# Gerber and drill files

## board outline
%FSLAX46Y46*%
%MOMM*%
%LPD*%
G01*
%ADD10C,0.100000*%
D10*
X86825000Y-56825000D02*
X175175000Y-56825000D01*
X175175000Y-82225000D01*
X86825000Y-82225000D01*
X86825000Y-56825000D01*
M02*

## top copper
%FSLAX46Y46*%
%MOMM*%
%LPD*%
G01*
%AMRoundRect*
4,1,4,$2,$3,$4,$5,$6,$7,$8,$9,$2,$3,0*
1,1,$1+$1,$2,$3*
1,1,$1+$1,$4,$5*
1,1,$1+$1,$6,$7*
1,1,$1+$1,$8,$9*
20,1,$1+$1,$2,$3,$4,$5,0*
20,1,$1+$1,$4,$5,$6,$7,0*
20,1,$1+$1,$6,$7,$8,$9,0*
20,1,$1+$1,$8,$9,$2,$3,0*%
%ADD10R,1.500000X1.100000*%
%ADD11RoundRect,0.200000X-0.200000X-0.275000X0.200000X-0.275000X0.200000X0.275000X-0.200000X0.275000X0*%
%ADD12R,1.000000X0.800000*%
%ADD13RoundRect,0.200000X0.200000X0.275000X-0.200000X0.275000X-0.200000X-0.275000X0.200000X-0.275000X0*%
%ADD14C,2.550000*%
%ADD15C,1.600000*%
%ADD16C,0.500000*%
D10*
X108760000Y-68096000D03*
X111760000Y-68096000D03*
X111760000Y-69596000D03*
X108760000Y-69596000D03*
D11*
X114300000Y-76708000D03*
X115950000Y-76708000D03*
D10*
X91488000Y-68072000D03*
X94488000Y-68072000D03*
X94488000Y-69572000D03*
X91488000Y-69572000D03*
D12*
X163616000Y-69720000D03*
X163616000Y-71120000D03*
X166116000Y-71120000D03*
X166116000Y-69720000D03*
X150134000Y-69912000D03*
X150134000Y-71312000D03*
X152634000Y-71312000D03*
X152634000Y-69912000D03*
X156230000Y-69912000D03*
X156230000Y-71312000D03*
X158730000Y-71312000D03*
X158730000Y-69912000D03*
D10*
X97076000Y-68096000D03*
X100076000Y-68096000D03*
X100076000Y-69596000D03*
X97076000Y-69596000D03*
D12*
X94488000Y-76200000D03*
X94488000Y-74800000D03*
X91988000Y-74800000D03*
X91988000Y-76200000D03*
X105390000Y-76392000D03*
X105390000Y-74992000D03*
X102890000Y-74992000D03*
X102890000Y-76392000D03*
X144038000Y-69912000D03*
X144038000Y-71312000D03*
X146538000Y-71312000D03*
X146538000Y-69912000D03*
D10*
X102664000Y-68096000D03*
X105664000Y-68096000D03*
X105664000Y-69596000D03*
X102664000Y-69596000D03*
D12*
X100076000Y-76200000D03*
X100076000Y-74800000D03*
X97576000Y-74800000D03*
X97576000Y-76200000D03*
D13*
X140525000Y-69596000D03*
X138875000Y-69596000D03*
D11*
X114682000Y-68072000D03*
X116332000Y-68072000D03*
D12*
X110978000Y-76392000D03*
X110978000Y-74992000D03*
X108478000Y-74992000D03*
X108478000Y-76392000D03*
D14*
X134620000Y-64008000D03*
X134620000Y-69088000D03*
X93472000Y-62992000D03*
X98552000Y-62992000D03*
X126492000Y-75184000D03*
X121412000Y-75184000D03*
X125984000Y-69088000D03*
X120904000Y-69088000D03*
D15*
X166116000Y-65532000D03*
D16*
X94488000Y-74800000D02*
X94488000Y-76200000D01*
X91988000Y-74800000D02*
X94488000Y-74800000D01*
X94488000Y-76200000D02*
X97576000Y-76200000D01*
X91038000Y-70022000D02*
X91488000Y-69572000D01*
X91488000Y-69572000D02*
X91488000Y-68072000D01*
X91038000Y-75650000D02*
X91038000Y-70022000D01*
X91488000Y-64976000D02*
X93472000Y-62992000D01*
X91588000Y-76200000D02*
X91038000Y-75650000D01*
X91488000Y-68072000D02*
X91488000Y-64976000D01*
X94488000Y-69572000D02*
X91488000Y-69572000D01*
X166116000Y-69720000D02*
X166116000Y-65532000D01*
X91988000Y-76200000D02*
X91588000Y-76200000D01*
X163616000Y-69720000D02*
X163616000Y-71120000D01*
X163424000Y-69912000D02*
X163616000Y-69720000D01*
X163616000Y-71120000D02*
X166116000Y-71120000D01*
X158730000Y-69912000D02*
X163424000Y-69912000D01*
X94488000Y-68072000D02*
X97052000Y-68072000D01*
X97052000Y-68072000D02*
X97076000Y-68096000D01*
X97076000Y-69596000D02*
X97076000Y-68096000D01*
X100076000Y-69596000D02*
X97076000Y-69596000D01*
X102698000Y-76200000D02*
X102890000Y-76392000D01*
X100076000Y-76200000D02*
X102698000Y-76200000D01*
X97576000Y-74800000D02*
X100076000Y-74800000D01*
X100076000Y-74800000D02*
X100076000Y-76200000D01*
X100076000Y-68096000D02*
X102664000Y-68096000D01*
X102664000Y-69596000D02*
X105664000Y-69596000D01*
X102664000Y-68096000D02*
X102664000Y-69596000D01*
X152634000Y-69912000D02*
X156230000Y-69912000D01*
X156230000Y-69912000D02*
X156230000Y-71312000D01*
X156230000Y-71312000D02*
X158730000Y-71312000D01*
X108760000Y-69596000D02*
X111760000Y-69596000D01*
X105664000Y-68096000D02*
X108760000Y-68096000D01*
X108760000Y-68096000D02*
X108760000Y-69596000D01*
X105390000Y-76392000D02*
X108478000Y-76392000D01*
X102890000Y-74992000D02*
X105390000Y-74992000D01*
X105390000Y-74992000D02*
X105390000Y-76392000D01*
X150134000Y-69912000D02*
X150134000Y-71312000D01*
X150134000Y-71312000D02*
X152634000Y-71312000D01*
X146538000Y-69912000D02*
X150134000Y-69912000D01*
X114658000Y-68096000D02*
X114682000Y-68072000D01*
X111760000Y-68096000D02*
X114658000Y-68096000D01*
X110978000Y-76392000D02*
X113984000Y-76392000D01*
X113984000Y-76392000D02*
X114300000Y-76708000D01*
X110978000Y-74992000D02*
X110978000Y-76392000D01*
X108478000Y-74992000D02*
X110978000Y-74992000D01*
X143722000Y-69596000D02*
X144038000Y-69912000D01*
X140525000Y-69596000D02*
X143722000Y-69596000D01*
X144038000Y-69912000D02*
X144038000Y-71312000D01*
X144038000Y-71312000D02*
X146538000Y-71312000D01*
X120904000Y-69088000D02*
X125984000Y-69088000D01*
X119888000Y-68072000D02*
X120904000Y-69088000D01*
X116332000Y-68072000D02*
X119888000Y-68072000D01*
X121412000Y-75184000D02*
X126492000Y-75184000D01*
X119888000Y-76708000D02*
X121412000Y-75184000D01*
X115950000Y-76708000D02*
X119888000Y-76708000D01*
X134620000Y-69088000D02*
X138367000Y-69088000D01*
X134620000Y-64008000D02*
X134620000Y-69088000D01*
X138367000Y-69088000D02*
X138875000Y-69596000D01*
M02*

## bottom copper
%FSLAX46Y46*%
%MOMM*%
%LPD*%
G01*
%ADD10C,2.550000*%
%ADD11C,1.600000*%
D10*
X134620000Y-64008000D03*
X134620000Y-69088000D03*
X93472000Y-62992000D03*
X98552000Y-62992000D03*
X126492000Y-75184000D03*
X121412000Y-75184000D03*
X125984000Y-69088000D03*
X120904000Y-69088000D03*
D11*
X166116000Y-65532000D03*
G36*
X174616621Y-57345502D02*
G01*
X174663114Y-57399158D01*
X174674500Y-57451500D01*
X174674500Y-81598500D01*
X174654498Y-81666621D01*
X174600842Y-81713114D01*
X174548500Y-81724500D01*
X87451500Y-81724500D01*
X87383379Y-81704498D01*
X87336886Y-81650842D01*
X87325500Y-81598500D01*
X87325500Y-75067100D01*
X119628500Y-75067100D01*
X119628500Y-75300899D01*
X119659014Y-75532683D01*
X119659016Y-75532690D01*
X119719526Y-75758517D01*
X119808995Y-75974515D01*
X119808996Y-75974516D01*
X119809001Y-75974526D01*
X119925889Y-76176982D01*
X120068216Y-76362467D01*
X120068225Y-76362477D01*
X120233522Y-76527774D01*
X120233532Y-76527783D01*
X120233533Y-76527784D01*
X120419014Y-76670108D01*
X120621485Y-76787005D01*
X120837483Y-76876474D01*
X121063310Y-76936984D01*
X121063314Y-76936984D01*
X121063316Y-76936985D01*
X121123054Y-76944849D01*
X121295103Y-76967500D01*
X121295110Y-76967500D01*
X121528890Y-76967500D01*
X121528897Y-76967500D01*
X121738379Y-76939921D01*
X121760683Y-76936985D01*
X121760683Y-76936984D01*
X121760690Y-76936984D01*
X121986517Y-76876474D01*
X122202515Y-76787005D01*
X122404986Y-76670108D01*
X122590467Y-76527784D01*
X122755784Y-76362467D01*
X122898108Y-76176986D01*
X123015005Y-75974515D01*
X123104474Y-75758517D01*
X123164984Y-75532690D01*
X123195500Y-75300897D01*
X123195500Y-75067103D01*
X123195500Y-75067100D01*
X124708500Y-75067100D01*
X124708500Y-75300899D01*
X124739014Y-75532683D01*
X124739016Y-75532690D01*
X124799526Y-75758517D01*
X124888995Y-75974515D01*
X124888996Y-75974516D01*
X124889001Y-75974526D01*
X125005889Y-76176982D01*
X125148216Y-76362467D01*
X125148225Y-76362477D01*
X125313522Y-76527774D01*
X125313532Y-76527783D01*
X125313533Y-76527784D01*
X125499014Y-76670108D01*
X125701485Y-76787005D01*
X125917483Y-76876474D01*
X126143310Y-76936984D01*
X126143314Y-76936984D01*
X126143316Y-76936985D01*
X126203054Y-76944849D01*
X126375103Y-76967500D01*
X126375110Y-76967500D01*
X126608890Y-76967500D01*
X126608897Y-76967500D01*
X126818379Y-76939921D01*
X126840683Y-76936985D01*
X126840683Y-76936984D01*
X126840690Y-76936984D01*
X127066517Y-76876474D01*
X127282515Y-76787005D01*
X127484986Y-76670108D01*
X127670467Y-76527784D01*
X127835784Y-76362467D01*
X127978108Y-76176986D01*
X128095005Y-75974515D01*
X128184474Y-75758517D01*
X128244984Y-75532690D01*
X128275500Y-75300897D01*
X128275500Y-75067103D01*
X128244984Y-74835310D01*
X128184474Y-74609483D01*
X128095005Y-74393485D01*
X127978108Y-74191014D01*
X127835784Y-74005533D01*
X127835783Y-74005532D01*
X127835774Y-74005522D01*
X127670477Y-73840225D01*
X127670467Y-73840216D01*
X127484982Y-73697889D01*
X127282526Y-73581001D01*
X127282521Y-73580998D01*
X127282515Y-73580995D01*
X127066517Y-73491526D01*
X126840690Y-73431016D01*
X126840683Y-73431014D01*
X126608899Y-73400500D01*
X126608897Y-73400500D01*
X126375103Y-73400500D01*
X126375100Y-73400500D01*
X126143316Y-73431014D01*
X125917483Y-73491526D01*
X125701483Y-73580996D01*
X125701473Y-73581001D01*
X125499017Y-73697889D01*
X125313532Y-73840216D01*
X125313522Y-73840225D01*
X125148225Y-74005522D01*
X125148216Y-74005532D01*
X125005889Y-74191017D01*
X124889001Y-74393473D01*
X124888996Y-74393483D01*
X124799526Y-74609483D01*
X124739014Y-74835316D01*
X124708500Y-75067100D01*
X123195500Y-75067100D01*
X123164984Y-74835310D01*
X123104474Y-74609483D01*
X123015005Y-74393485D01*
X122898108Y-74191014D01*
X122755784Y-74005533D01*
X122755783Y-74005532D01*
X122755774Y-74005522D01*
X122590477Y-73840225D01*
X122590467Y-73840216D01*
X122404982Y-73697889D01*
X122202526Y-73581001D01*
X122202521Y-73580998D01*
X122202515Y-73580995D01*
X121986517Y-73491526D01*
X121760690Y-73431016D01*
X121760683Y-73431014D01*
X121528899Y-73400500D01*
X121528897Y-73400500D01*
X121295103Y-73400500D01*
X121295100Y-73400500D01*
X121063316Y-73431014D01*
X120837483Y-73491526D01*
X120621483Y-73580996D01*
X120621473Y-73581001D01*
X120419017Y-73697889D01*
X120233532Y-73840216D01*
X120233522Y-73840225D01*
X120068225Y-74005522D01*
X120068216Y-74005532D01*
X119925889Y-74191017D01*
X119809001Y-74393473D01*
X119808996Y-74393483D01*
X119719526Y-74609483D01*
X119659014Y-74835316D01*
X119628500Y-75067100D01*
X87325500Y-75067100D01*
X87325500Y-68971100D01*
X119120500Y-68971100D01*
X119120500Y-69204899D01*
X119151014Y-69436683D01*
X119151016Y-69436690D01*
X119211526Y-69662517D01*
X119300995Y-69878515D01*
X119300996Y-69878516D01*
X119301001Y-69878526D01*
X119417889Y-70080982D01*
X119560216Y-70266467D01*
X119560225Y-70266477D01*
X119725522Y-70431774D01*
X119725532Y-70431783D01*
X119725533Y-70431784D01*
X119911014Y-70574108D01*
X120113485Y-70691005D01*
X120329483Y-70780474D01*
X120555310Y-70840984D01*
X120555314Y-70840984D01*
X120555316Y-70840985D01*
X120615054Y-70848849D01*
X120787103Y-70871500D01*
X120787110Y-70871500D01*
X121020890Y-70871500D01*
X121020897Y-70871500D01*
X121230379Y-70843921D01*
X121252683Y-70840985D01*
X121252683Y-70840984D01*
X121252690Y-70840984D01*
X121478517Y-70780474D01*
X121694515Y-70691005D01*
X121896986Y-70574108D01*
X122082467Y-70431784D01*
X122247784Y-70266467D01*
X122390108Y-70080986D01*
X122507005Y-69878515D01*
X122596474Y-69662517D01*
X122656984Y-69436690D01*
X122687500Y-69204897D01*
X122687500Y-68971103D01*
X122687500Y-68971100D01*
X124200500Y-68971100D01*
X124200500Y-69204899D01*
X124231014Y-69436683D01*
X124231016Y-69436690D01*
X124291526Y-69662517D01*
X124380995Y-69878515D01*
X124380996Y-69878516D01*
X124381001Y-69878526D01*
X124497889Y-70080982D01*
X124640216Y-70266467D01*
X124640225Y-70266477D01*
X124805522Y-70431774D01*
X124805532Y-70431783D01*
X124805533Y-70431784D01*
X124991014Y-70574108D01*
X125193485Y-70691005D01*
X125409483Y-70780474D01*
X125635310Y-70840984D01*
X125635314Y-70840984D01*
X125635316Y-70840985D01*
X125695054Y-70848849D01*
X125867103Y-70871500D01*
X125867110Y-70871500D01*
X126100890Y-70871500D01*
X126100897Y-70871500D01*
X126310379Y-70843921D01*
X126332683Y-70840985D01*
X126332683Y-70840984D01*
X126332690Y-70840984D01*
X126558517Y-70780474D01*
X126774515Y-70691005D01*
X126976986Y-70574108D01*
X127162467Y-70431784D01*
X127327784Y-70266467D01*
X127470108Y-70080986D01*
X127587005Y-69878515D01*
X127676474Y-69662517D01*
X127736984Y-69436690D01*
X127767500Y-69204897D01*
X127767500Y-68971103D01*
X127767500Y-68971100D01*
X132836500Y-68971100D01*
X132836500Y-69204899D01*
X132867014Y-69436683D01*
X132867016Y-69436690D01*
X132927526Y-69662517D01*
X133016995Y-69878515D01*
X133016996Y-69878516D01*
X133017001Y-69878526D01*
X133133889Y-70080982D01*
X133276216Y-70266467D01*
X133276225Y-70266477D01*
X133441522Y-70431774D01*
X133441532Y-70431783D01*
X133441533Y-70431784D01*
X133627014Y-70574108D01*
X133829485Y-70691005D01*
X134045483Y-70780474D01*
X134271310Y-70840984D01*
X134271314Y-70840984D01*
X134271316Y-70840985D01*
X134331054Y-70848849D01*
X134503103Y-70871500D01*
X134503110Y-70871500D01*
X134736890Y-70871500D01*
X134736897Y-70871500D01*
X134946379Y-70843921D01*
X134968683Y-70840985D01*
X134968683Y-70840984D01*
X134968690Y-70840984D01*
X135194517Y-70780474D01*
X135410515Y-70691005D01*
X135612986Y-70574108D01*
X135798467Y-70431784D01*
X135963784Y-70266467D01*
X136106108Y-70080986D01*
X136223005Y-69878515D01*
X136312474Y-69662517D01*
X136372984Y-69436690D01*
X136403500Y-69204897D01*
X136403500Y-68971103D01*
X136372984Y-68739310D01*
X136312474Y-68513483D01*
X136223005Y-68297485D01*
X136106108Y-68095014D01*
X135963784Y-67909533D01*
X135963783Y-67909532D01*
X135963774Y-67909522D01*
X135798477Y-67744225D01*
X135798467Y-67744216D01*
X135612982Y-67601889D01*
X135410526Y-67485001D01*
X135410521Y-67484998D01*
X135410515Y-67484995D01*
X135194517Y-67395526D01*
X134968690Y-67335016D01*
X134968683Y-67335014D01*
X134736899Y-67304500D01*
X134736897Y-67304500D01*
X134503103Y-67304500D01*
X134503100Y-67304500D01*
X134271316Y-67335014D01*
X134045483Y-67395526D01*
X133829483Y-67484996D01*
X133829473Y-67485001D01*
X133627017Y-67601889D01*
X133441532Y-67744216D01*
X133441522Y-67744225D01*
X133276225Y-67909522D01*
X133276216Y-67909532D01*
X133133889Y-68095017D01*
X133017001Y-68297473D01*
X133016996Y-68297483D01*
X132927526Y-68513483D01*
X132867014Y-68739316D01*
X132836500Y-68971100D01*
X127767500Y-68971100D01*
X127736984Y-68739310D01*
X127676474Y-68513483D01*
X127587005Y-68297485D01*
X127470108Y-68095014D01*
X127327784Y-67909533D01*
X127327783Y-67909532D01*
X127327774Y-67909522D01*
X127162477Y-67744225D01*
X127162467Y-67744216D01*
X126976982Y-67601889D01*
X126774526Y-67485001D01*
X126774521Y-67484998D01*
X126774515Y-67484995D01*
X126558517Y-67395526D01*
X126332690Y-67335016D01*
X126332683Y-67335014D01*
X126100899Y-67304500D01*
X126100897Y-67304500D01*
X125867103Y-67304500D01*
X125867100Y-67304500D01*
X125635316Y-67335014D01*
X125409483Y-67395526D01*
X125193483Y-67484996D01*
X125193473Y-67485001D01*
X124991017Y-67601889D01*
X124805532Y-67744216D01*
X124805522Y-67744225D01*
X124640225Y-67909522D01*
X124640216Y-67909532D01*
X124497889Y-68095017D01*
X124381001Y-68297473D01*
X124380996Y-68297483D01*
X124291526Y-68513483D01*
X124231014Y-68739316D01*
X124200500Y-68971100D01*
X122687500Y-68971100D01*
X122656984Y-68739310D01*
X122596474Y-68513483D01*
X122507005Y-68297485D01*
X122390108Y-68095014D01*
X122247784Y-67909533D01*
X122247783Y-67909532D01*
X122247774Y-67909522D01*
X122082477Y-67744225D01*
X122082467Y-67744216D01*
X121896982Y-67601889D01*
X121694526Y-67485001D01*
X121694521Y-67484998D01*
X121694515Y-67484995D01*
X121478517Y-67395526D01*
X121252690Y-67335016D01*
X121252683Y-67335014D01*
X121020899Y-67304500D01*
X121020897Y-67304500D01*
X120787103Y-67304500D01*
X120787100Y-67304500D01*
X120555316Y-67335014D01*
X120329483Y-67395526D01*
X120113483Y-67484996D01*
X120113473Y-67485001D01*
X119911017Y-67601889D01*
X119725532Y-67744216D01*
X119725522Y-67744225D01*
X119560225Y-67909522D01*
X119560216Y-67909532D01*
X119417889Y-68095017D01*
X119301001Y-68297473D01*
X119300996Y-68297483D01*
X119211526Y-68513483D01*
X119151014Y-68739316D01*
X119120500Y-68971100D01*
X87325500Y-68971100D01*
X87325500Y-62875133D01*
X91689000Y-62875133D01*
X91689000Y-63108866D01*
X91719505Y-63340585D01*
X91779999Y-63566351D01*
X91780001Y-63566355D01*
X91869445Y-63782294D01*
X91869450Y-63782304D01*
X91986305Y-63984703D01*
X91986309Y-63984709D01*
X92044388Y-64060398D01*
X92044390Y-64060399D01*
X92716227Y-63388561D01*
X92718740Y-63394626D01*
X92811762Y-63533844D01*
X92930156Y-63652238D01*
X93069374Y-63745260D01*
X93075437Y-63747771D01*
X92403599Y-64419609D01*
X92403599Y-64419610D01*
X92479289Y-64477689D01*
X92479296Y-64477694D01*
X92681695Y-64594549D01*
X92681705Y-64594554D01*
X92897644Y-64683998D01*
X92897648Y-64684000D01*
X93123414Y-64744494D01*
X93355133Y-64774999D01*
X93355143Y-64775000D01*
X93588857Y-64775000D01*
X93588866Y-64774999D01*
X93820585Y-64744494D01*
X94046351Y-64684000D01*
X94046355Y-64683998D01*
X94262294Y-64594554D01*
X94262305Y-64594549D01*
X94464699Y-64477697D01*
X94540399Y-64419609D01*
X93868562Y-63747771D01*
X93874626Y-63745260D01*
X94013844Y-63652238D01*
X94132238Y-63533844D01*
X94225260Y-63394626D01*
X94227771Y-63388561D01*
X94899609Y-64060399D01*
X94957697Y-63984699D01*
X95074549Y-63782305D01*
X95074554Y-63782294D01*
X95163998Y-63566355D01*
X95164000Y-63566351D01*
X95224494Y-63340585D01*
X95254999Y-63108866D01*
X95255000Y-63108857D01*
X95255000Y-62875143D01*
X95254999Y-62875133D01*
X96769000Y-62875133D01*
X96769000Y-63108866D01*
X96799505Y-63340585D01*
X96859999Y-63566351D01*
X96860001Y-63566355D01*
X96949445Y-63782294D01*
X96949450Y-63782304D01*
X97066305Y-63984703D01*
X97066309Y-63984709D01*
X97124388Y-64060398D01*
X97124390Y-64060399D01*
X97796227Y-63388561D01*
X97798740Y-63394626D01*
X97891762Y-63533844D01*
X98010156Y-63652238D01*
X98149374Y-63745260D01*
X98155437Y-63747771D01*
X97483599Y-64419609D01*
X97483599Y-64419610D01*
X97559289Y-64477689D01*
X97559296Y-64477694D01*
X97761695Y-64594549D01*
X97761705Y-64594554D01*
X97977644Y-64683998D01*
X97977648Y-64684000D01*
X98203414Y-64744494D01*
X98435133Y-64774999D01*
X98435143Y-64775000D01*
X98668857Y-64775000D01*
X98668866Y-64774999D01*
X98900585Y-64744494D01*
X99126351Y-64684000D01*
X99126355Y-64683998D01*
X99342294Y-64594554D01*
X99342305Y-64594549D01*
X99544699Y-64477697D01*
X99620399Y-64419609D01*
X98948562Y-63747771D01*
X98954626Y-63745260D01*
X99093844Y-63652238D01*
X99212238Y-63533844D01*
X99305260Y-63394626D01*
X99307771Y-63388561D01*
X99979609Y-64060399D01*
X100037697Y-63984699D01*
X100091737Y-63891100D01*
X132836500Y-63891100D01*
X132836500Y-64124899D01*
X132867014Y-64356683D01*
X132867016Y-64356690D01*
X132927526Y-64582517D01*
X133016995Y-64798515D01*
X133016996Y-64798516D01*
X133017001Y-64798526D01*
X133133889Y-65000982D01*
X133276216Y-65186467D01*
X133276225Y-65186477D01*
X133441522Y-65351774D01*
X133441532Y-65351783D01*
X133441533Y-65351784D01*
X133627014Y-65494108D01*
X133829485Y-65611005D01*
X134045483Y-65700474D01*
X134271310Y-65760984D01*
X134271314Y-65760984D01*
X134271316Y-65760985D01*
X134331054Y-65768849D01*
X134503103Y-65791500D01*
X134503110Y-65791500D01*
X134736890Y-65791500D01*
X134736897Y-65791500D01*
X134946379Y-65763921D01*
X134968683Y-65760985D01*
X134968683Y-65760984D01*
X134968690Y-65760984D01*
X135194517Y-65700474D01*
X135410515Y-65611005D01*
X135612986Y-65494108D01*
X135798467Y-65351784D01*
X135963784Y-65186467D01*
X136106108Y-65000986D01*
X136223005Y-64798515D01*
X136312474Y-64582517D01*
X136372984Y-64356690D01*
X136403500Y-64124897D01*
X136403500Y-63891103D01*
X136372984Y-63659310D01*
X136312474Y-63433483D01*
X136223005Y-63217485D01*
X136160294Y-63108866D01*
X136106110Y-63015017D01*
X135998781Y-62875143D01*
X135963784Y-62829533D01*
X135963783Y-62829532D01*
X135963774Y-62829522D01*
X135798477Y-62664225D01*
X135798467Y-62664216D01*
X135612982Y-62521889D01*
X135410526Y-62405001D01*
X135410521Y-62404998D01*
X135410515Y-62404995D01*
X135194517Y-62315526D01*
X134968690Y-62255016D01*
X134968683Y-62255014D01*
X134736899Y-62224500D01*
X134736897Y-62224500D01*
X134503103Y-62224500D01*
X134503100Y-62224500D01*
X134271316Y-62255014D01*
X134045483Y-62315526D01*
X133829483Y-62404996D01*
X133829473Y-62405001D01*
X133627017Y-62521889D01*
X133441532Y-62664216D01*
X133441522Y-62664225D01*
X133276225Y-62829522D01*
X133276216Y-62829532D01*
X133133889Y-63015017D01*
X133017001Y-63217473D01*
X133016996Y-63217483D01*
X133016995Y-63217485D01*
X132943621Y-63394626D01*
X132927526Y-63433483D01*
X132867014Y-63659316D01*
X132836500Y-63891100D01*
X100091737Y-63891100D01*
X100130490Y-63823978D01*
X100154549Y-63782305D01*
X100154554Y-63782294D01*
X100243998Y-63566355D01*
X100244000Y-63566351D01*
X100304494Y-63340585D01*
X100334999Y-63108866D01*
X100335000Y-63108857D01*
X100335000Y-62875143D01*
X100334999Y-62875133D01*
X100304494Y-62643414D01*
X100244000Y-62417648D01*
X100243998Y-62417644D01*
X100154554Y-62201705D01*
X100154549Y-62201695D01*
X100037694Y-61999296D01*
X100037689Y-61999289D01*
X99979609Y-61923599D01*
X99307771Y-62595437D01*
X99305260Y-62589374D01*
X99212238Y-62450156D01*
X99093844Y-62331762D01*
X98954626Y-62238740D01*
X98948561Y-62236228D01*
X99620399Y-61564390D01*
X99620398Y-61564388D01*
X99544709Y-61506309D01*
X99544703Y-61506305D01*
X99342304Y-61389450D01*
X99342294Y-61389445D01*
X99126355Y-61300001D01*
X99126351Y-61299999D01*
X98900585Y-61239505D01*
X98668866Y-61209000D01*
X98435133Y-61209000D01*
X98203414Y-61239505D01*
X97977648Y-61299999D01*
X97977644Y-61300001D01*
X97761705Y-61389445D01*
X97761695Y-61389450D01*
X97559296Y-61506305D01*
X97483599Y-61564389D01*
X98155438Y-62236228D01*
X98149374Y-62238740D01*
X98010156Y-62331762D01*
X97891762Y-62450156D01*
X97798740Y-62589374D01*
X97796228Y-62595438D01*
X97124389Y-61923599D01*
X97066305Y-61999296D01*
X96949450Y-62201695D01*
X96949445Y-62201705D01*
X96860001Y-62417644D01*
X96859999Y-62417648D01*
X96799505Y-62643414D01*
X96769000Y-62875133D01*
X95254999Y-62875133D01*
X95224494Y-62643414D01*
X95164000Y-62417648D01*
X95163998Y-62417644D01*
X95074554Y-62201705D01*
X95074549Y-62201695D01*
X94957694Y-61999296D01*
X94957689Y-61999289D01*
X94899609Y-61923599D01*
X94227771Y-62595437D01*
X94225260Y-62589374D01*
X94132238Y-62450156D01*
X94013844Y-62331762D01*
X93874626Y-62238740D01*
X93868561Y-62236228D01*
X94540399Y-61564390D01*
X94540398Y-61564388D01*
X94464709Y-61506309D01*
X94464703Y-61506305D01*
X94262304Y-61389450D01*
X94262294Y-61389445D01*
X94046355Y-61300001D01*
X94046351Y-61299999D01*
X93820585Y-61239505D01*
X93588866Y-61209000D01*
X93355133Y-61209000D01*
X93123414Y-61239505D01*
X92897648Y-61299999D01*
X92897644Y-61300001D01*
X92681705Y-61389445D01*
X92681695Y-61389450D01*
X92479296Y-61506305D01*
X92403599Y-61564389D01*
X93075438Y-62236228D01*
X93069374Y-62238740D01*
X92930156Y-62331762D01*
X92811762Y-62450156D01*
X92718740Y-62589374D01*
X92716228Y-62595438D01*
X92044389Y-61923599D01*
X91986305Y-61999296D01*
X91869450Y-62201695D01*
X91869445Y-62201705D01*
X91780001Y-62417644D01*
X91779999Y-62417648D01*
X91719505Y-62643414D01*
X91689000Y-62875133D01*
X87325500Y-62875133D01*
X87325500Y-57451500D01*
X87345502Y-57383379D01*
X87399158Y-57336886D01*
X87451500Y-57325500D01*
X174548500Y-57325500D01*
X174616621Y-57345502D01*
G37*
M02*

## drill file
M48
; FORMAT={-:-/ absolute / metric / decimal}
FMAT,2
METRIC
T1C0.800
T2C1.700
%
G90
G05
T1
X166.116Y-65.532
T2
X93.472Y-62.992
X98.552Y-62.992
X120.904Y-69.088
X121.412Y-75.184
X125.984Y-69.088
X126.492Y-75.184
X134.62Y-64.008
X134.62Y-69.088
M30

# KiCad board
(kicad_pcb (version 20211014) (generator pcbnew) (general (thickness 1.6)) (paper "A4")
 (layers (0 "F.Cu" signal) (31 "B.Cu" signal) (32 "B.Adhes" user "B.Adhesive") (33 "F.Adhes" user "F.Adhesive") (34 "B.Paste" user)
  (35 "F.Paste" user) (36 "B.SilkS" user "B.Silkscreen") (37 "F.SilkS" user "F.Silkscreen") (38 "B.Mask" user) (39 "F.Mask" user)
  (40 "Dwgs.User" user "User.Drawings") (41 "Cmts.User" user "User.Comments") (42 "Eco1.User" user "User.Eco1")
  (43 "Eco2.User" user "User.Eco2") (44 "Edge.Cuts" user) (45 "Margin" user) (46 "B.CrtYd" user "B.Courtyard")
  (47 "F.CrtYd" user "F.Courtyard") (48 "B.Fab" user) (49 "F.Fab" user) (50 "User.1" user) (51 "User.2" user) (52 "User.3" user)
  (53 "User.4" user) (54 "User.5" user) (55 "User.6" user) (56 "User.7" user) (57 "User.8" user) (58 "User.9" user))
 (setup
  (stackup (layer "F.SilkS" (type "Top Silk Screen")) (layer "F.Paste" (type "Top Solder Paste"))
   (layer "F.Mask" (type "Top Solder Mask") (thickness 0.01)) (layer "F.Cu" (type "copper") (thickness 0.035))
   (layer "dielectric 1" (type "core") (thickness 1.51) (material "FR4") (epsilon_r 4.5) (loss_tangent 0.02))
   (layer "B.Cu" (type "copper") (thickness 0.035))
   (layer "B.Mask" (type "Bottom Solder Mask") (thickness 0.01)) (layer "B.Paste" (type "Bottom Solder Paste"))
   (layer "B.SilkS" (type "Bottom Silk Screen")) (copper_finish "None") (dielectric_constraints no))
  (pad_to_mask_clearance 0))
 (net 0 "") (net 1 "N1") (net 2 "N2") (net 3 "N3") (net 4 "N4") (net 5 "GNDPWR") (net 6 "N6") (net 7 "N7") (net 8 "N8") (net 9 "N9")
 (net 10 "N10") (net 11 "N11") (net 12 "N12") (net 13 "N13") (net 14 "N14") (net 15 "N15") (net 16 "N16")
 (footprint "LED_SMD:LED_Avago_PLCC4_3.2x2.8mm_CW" (layer "F.Cu") (at 110.26 68.846)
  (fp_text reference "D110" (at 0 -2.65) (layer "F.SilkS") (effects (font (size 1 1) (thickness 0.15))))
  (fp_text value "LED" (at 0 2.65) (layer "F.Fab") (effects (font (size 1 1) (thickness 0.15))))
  (pad "1" smd rect (at -1.5 -0.75) (size 1.5 1.1) (layers "F.Cu" "F.Paste" "F.Mask") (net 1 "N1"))
  (pad "2" smd rect (at 1.5 -0.75) (size 1.5 1.1) (layers "F.Cu" "F.Paste" "F.Mask") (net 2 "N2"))
  (pad "3" smd rect (at 1.5 0.75) (size 1.5 1.1) (layers "F.Cu" "F.Paste" "F.Mask") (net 1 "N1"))
  (pad "4" smd rect (at -1.5 0.75) (size 1.5 1.1) (layers "F.Cu" "F.Paste" "F.Mask") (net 1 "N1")))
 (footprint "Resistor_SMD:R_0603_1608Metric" (layer "F.Cu") (at 115.125 76.708)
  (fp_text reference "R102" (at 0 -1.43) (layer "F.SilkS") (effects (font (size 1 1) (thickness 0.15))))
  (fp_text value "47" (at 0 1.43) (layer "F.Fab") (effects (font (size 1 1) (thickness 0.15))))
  (pad "1" smd roundrect (at -0.825 0) (size 0.8 0.95) (layers "F.Cu" "F.Paste" "F.Mask") (roundrect_rratio 0.25) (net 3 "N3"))
  (pad "2" smd roundrect (at 0.825 0) (size 0.8 0.95) (layers "F.Cu" "F.Paste" "F.Mask") (roundrect_rratio 0.25) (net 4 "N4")))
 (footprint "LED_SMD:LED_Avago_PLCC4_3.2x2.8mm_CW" (layer "F.Cu") (at 92.988 68.822)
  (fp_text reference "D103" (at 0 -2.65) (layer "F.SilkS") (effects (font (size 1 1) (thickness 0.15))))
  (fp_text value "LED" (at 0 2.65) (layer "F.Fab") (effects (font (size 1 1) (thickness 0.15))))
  (pad "1" smd rect (at -1.5 -0.75) (size 1.5 1.1) (layers "F.Cu" "F.Paste" "F.Mask") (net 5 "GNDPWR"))
  (pad "2" smd rect (at 1.5 -0.75) (size 1.5 1.1) (layers "F.Cu" "F.Paste" "F.Mask") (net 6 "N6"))
  (pad "3" smd rect (at 1.5 0.75) (size 1.5 1.1) (layers "F.Cu" "F.Paste" "F.Mask") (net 5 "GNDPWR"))
  (pad "4" smd rect (at -1.5 0.75) (size 1.5 1.1) (layers "F.Cu" "F.Paste" "F.Mask") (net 5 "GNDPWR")))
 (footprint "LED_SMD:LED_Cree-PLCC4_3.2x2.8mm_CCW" (layer "F.Cu") (at 164.866 70.42)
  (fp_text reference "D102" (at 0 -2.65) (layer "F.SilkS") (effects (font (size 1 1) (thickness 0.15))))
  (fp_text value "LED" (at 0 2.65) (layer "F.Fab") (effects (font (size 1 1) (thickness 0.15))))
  (pad "1" smd rect (at -1.25 -0.7) (size 1 0.8) (layers "F.Cu" "F.Paste" "F.Mask") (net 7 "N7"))
  (pad "2" smd rect (at -1.25 0.7) (size 1 0.8) (layers "F.Cu" "F.Paste" "F.Mask") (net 7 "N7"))
  (pad "3" smd rect (at 1.25 0.7) (size 1 0.8) (layers "F.Cu" "F.Paste" "F.Mask") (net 7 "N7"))
  (pad "4" smd rect (at 1.25 -0.7) (size 1 0.8) (layers "F.Cu" "F.Paste" "F.Mask") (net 5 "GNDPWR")))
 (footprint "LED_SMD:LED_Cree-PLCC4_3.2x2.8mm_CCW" (layer "F.Cu") (at 151.384 70.612)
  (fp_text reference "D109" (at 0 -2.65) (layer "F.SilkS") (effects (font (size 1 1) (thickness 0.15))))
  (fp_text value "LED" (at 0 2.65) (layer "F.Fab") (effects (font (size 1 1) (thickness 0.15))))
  (pad "1" smd rect (at -1.25 -0.7) (size 1 0.8) (layers "F.Cu" "F.Paste" "F.Mask") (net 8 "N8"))
  (pad "2" smd rect (at -1.25 0.7) (size 1 0.8) (layers "F.Cu" "F.Paste" "F.Mask") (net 8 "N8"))
  (pad "3" smd rect (at 1.25 0.7) (size 1 0.8) (layers "F.Cu" "F.Paste" "F.Mask") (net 8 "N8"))
  (pad "4" smd rect (at 1.25 -0.7) (size 1 0.8) (layers "F.Cu" "F.Paste" "F.Mask") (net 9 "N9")))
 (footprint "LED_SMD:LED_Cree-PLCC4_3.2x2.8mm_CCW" (layer "F.Cu") (at 157.48 70.612)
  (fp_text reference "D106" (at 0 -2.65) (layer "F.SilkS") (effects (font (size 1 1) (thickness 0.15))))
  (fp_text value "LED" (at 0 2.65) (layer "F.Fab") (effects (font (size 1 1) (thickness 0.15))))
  (pad "1" smd rect (at -1.25 -0.7) (size 1 0.8) (layers "F.Cu" "F.Paste" "F.Mask") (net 9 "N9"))
  (pad "2" smd rect (at -1.25 0.7) (size 1 0.8) (layers "F.Cu" "F.Paste" "F.Mask") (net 9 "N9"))
  (pad "3" smd rect (at 1.25 0.7) (size 1 0.8) (layers "F.Cu" "F.Paste" "F.Mask") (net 9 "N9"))
  (pad "4" smd rect (at 1.25 -0.7) (size 1 0.8) (layers "F.Cu" "F.Paste" "F.Mask") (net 7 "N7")))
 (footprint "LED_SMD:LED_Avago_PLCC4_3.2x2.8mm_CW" (layer "F.Cu") (at 98.576 68.846)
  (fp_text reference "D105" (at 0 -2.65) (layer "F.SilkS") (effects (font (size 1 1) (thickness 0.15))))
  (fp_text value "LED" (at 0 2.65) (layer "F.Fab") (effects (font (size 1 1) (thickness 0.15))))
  (pad "1" smd rect (at -1.5 -0.75) (size 1.5 1.1) (layers "F.Cu" "F.Paste" "F.Mask") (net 6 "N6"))
  (pad "2" smd rect (at 1.5 -0.75) (size 1.5 1.1) (layers "F.Cu" "F.Paste" "F.Mask") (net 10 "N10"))
  (pad "3" smd rect (at 1.5 0.75) (size 1.5 1.1) (layers "F.Cu" "F.Paste" "F.Mask") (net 6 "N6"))
  (pad "4" smd rect (at -1.5 0.75) (size 1.5 1.1) (layers "F.Cu" "F.Paste" "F.Mask") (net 6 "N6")))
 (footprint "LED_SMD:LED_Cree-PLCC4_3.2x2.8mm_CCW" (layer "F.Cu") (at 93.238 75.5 180)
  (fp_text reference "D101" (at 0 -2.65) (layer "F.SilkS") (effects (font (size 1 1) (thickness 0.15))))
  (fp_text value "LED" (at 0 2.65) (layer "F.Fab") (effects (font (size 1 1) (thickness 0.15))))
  (pad "1" smd rect (at -1.25 -0.7 180) (size 1 0.8) (layers "F.Cu" "F.Paste" "F.Mask") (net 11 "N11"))
  (pad "2" smd rect (at -1.25 0.7 180) (size 1 0.8) (layers "F.Cu" "F.Paste" "F.Mask") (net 11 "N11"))
  (pad "3" smd rect (at 1.25 0.7 180) (size 1 0.8) (layers "F.Cu" "F.Paste" "F.Mask") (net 11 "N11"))
  (pad "4" smd rect (at 1.25 -0.7 180) (size 1 0.8) (layers "F.Cu" "F.Paste" "F.Mask") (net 5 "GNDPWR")))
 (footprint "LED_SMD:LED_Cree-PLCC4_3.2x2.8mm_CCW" (layer "F.Cu") (at 104.14 75.692 180)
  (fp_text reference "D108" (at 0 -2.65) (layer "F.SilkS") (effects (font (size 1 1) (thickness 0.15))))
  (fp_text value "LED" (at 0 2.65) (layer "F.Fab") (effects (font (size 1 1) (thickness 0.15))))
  (pad "1" smd rect (at -1.25 -0.7 180) (size 1 0.8) (layers "F.Cu" "F.Paste" "F.Mask") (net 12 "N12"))
  (pad "2" smd rect (at -1.25 0.7 180) (size 1 0.8) (layers "F.Cu" "F.Paste" "F.Mask") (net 12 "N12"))
  (pad "3" smd rect (at 1.25 0.7 180) (size 1 0.8) (layers "F.Cu" "F.Paste" "F.Mask") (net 12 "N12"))
  (pad "4" smd rect (at 1.25 -0.7 180) (size 1 0.8) (layers "F.Cu" "F.Paste" "F.Mask") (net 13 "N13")))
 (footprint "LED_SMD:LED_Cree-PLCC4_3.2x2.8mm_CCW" (layer "F.Cu") (at 145.288 70.612)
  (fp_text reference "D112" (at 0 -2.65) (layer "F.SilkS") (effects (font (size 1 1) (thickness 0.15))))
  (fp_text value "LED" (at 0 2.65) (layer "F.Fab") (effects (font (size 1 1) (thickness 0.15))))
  (pad "1" smd rect (at -1.25 -0.7) (size 1 0.8) (layers "F.Cu" "F.Paste" "F.Mask") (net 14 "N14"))
  (pad "2" smd rect (at -1.25 0.7) (size 1 0.8) (layers "F.Cu" "F.Paste" "F.Mask") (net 14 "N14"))
  (pad "3" smd rect (at 1.25 0.7) (size 1 0.8) (layers "F.Cu" "F.Paste" "F.Mask") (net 14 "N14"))
  (pad "4" smd rect (at 1.25 -0.7) (size 1 0.8) (layers "F.Cu" "F.Paste" "F.Mask") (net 8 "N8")))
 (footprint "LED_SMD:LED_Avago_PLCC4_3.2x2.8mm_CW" (layer "F.Cu") (at 104.164 68.846)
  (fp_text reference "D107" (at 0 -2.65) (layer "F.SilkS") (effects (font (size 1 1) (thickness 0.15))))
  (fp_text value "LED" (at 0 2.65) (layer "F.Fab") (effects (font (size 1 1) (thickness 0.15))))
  (pad "1" smd rect (at -1.5 -0.75) (size 1.5 1.1) (layers "F.Cu" "F.Paste" "F.Mask") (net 10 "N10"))
  (pad "2" smd rect (at 1.5 -0.75) (size 1.5 1.1) (layers "F.Cu" "F.Paste" "F.Mask") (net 1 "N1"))
  (pad "3" smd rect (at 1.5 0.75) (size 1.5 1.1) (layers "F.Cu" "F.Paste" "F.Mask") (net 10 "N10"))
  (pad "4" smd rect (at -1.5 0.75) (size 1.5 1.1) (layers "F.Cu" "F.Paste" "F.Mask") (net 10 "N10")))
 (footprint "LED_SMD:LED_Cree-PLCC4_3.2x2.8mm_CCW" (layer "F.Cu") (at 98.826 75.5 180)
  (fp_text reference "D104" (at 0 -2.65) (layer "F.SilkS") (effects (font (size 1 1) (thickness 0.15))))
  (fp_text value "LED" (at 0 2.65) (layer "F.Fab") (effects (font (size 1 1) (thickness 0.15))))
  (pad "1" smd rect (at -1.25 -0.7 180) (size 1 0.8) (layers "F.Cu" "F.Paste" "F.Mask") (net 13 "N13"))
  (pad "2" smd rect (at -1.25 0.7 180) (size 1 0.8) (layers "F.Cu" "F.Paste" "F.Mask") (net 13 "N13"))
  (pad "3" smd rect (at 1.25 0.7 180) (size 1 0.8) (layers "F.Cu" "F.Paste" "F.Mask") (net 13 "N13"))
  (pad "4" smd rect (at 1.25 -0.7 180) (size 1 0.8) (layers "F.Cu" "F.Paste" "F.Mask") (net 11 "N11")))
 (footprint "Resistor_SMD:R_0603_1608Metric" (layer "F.Cu") (at 139.7 69.596 180)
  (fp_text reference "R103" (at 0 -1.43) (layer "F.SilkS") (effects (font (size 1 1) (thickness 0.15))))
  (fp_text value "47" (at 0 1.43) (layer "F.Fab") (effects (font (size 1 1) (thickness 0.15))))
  (pad "1" smd roundrect (at -0.825 0 180) (size 0.8 0.95) (layers "F.Cu" "F.Paste" "F.Mask") (roundrect_rratio 0.25) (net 14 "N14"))
  (pad "2" smd roundrect (at 0.825 0 180) (size 0.8 0.95) (layers "F.Cu" "F.Paste" "F.Mask") (roundrect_rratio 0.25) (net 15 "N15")))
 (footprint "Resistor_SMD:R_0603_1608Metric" (layer "F.Cu") (at 115.507 68.072)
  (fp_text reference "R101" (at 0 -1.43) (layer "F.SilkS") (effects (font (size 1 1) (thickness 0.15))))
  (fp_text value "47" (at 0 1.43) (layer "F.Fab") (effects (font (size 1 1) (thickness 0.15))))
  (pad "1" smd roundrect (at -0.825 0) (size 0.8 0.95) (layers "F.Cu" "F.Paste" "F.Mask") (roundrect_rratio 0.25) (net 2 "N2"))
  (pad "2" smd roundrect (at 0.825 0) (size 0.8 0.95) (layers "F.Cu" "F.Paste" "F.Mask") (roundrect_rratio 0.25) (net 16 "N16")))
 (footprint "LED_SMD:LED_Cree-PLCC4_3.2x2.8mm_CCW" (layer "F.Cu") (at 109.728 75.692 180)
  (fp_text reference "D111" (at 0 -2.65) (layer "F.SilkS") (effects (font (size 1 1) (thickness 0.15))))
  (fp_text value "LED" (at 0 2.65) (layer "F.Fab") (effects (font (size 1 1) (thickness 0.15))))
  (pad "1" smd rect (at -1.25 -0.7 180) (size 1 0.8) (layers "F.Cu" "F.Paste" "F.Mask") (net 3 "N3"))
  (pad "2" smd rect (at -1.25 0.7 180) (size 1 0.8) (layers "F.Cu" "F.Paste" "F.Mask") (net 3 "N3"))
  (pad "3" smd rect (at 1.25 0.7 180) (size 1 0.8) (layers "F.Cu" "F.Paste" "F.Mask") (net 3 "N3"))
  (pad "4" smd rect (at 1.25 -0.7 180) (size 1 0.8) (layers "F.Cu" "F.Paste" "F.Mask") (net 12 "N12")))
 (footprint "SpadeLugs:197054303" (layer "B.Cu") (at 134.62 64.008 -90)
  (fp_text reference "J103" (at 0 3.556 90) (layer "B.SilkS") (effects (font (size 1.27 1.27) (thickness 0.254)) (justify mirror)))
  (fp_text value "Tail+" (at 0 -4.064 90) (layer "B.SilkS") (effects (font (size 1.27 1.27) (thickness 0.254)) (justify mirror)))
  (pad "1" thru_hole circle locked (at 0 0 270) (size 2.55 2.55) (drill 1.7) (layers *.Cu *.Mask) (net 15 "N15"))
  (pad "2" thru_hole circle locked (at 5.08 0 270) (size 2.55 2.55) (drill 1.7) (layers *.Cu *.Mask) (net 15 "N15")))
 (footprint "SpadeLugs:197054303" (layer "B.Cu") (at 93.472 62.992)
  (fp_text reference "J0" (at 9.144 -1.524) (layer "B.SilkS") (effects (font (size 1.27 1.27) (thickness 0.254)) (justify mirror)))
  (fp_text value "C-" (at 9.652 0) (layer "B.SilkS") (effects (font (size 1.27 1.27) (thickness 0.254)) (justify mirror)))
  (pad "1" thru_hole circle locked (at 0 0) (size 2.55 2.55) (drill 1.7) (layers *.Cu *.Mask) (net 5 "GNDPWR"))
  (pad "2" thru_hole circle locked (at 5.08 0) (size 2.55 2.55) (drill 1.7) (layers *.Cu *.Mask) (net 5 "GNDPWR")))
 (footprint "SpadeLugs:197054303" (layer "B.Cu") (at 126.492 75.184 180)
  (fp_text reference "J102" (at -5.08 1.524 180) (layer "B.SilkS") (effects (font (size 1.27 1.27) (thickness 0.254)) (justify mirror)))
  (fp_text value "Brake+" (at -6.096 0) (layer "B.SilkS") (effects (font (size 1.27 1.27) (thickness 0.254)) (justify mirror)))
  (pad "1" thru_hole circle locked (at 0 0 180) (size 2.55 2.55) (drill 1.7) (layers *.Cu *.Mask) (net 4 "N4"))
  (pad "2" thru_hole circle locked (at 5.08 0 180) (size 2.55 2.55) (drill 1.7) (layers *.Cu *.Mask) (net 4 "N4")))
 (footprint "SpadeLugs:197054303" (layer "B.Cu") (at 125.984 69.088 180)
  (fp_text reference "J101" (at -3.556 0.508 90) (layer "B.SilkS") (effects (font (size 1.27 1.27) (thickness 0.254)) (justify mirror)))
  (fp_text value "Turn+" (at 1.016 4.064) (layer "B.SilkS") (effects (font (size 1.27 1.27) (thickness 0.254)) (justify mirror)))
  (pad "1" thru_hole circle locked (at 0 0 180) (size 2.55 2.55) (drill 1.7) (layers *.Cu *.Mask) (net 16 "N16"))
  (pad "2" thru_hole circle locked (at 5.08 0 180) (size 2.55 2.55) (drill 1.7) (layers *.Cu *.Mask) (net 16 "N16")))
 (gr_rect (start 86.825 56.825) (end 175.175 82.225) (layer "Edge.Cuts") (width 0.1) (fill none))
 (segment (start 94.488 74.8) (end 94.488 76.2) (width 0.5) (layer "F.Cu") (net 11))
 (segment (start 91.988 74.8) (end 94.488 74.8) (width 0.5) (layer "F.Cu") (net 11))
 (segment (start 94.488 76.2) (end 97.576 76.2) (width 0.5) (layer "F.Cu") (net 11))
 (segment (start 91.038 70.022) (end 91.488 69.572) (width 0.5) (layer "F.Cu") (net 5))
 (segment (start 91.488 69.572) (end 91.488 68.072) (width 0.5) (layer "F.Cu") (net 5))
 (segment (start 91.038 75.65) (end 91.038 70.022) (width 0.5) (layer "F.Cu") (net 5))
 (segment (start 91.488 64.976) (end 93.472 62.992) (width 0.5) (layer "F.Cu") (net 5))
 (segment (start 91.588 76.2) (end 91.038 75.65) (width 0.5) (layer "F.Cu") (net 5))
 (segment (start 91.488 68.072) (end 91.488 64.976) (width 0.5) (layer "F.Cu") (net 5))
 (segment (start 94.488 69.572) (end 91.488 69.572) (width 0.5) (layer "F.Cu") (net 5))
 (segment (start 166.116 69.72) (end 166.116 65.532) (width 0.5) (layer "F.Cu") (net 5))
 (segment (start 91.988 76.2) (end 91.588 76.2) (width 0.5) (layer "F.Cu") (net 5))
 (via (at 166.116 65.532) (size 1.6) (drill 0.8) (layers "F.Cu" "B.Cu") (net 5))
 (segment (start 163.616 69.72) (end 163.616 71.12) (width 0.5) (layer "F.Cu") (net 7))
 (segment (start 163.424 69.912) (end 163.616 69.72) (width 0.5) (layer "F.Cu") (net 7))
 (segment (start 163.616 71.12) (end 166.116 71.12) (width 0.5) (layer "F.Cu") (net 7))
 (segment (start 158.73 69.912) (end 163.424 69.912) (width 0.5) (layer "F.Cu") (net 7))
 (segment (start 94.488 68.072) (end 97.052 68.072) (width 0.5) (layer "F.Cu") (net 6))
 (segment (start 97.052 68.072) (end 97.076 68.096) (width 0.5) (layer "F.Cu") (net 6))
 (segment (start 97.076 69.596) (end 97.076 68.096) (width 0.5) (layer "F.Cu") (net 6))
 (segment (start 100.076 69.596) (end 97.076 69.596) (width 0.5) (layer "F.Cu") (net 6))
 (segment (start 102.698 76.2) (end 102.89 76.392) (width 0.5) (layer "F.Cu") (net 13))
 (segment (start 100.076 76.2) (end 102.698 76.2) (width 0.5) (layer "F.Cu") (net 13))
 (segment (start 97.576 74.8) (end 100.076 74.8) (width 0.5) (layer "F.Cu") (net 13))
 (segment (start 100.076 74.8) (end 100.076 76.2) (width 0.5) (layer "F.Cu") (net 13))
 (segment (start 100.076 68.096) (end 102.664 68.096) (width 0.5) (layer "F.Cu") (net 10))
 (segment (start 102.664 69.596) (end 105.664 69.596) (width 0.5) (layer "F.Cu") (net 10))
 (segment (start 102.664 68.096) (end 102.664 69.596) (width 0.5) (layer "F.Cu") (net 10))
 (segment (start 152.634 69.912) (end 156.23 69.912) (width 0.5) (layer "F.Cu") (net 9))
 (segment (start 156.23 69.912) (end 156.23 71.312) (width 0.5) (layer "F.Cu") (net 9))
 (segment (start 156.23 71.312) (end 158.73 71.312) (width 0.5) (layer "F.Cu") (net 9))
 (segment (start 108.76 69.596) (end 111.76 69.596) (width 0.5) (layer "F.Cu") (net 1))
 (segment (start 105.664 68.096) (end 108.76 68.096) (width 0.5) (layer "F.Cu") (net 1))
 (segment (start 108.76 68.096) (end 108.76 69.596) (width 0.5) (layer "F.Cu") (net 1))
 (segment (start 105.39 76.392) (end 108.478 76.392) (width 0.5) (layer "F.Cu") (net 12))
 (segment (start 102.89 74.992) (end 105.39 74.992) (width 0.5) (layer "F.Cu") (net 12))
 (segment (start 105.39 74.992) (end 105.39 76.392) (width 0.5) (layer "F.Cu") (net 12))
 (segment (start 150.134 69.912) (end 150.134 71.312) (width 0.5) (layer "F.Cu") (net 8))
 (segment (start 150.134 71.312) (end 152.634 71.312) (width 0.5) (layer "F.Cu") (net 8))
 (segment (start 146.538 69.912) (end 150.134 69.912) (width 0.5) (layer "F.Cu") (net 8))
 (segment (start 114.658 68.096) (end 114.682 68.072) (width 0.5) (layer "F.Cu") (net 2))
 (segment (start 111.76 68.096) (end 114.658 68.096) (width 0.5) (layer "F.Cu") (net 2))
 (segment (start 110.978 76.392) (end 113.984 76.392) (width 0.5) (layer "F.Cu") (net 3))
 (segment (start 113.984 76.392) (end 114.3 76.708) (width 0.5) (layer "F.Cu") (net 3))
 (segment (start 110.978 74.992) (end 110.978 76.392) (width 0.5) (layer "F.Cu") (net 3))
 (segment (start 108.478 74.992) (end 110.978 74.992) (width 0.5) (layer "F.Cu") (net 3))
 (segment (start 143.722 69.596) (end 144.038 69.912) (width 0.5) (layer "F.Cu") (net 14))
 (segment (start 140.525 69.596) (end 143.722 69.596) (width 0.5) (layer "F.Cu") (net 14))
 (segment (start 144.038 69.912) (end 144.038 71.312) (width 0.5) (layer "F.Cu") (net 14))
 (segment (start 144.038 71.312) (end 146.538 71.312) (width 0.5) (layer "F.Cu") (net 14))
 (segment (start 120.904 69.088) (end 125.984 69.088) (width 0.5) (layer "F.Cu") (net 16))
 (segment (start 119.888 68.072) (end 120.904 69.088) (width 0.5) (layer "F.Cu") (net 16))
 (segment (start 116.332 68.072) (end 119.888 68.072) (width 0.5) (layer "F.Cu") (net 16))
 (segment (start 121.412 75.184) (end 126.492 75.184) (width 0.5) (layer "F.Cu") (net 4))
 (segment (start 119.888 76.708) (end 121.412 75.184) (width 0.5) (layer "F.Cu") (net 4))
 (segment (start 115.95 76.708) (end 119.888 76.708) (width 0.5) (layer "F.Cu") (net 4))
 (segment (start 134.62 69.088) (end 138.367 69.088) (width 0.5) (layer "F.Cu") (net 15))
 (segment (start 134.62 64.008) (end 134.62 69.088) (width 0.5) (layer "F.Cu") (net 15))
 (segment (start 138.367 69.088) (end 138.875 69.596) (width 0.5) (layer "F.Cu") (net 15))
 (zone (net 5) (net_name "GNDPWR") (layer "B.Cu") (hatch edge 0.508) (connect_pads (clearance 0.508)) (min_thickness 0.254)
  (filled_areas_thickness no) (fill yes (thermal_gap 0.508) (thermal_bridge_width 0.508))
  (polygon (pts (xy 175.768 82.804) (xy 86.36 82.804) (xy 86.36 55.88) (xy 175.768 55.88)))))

